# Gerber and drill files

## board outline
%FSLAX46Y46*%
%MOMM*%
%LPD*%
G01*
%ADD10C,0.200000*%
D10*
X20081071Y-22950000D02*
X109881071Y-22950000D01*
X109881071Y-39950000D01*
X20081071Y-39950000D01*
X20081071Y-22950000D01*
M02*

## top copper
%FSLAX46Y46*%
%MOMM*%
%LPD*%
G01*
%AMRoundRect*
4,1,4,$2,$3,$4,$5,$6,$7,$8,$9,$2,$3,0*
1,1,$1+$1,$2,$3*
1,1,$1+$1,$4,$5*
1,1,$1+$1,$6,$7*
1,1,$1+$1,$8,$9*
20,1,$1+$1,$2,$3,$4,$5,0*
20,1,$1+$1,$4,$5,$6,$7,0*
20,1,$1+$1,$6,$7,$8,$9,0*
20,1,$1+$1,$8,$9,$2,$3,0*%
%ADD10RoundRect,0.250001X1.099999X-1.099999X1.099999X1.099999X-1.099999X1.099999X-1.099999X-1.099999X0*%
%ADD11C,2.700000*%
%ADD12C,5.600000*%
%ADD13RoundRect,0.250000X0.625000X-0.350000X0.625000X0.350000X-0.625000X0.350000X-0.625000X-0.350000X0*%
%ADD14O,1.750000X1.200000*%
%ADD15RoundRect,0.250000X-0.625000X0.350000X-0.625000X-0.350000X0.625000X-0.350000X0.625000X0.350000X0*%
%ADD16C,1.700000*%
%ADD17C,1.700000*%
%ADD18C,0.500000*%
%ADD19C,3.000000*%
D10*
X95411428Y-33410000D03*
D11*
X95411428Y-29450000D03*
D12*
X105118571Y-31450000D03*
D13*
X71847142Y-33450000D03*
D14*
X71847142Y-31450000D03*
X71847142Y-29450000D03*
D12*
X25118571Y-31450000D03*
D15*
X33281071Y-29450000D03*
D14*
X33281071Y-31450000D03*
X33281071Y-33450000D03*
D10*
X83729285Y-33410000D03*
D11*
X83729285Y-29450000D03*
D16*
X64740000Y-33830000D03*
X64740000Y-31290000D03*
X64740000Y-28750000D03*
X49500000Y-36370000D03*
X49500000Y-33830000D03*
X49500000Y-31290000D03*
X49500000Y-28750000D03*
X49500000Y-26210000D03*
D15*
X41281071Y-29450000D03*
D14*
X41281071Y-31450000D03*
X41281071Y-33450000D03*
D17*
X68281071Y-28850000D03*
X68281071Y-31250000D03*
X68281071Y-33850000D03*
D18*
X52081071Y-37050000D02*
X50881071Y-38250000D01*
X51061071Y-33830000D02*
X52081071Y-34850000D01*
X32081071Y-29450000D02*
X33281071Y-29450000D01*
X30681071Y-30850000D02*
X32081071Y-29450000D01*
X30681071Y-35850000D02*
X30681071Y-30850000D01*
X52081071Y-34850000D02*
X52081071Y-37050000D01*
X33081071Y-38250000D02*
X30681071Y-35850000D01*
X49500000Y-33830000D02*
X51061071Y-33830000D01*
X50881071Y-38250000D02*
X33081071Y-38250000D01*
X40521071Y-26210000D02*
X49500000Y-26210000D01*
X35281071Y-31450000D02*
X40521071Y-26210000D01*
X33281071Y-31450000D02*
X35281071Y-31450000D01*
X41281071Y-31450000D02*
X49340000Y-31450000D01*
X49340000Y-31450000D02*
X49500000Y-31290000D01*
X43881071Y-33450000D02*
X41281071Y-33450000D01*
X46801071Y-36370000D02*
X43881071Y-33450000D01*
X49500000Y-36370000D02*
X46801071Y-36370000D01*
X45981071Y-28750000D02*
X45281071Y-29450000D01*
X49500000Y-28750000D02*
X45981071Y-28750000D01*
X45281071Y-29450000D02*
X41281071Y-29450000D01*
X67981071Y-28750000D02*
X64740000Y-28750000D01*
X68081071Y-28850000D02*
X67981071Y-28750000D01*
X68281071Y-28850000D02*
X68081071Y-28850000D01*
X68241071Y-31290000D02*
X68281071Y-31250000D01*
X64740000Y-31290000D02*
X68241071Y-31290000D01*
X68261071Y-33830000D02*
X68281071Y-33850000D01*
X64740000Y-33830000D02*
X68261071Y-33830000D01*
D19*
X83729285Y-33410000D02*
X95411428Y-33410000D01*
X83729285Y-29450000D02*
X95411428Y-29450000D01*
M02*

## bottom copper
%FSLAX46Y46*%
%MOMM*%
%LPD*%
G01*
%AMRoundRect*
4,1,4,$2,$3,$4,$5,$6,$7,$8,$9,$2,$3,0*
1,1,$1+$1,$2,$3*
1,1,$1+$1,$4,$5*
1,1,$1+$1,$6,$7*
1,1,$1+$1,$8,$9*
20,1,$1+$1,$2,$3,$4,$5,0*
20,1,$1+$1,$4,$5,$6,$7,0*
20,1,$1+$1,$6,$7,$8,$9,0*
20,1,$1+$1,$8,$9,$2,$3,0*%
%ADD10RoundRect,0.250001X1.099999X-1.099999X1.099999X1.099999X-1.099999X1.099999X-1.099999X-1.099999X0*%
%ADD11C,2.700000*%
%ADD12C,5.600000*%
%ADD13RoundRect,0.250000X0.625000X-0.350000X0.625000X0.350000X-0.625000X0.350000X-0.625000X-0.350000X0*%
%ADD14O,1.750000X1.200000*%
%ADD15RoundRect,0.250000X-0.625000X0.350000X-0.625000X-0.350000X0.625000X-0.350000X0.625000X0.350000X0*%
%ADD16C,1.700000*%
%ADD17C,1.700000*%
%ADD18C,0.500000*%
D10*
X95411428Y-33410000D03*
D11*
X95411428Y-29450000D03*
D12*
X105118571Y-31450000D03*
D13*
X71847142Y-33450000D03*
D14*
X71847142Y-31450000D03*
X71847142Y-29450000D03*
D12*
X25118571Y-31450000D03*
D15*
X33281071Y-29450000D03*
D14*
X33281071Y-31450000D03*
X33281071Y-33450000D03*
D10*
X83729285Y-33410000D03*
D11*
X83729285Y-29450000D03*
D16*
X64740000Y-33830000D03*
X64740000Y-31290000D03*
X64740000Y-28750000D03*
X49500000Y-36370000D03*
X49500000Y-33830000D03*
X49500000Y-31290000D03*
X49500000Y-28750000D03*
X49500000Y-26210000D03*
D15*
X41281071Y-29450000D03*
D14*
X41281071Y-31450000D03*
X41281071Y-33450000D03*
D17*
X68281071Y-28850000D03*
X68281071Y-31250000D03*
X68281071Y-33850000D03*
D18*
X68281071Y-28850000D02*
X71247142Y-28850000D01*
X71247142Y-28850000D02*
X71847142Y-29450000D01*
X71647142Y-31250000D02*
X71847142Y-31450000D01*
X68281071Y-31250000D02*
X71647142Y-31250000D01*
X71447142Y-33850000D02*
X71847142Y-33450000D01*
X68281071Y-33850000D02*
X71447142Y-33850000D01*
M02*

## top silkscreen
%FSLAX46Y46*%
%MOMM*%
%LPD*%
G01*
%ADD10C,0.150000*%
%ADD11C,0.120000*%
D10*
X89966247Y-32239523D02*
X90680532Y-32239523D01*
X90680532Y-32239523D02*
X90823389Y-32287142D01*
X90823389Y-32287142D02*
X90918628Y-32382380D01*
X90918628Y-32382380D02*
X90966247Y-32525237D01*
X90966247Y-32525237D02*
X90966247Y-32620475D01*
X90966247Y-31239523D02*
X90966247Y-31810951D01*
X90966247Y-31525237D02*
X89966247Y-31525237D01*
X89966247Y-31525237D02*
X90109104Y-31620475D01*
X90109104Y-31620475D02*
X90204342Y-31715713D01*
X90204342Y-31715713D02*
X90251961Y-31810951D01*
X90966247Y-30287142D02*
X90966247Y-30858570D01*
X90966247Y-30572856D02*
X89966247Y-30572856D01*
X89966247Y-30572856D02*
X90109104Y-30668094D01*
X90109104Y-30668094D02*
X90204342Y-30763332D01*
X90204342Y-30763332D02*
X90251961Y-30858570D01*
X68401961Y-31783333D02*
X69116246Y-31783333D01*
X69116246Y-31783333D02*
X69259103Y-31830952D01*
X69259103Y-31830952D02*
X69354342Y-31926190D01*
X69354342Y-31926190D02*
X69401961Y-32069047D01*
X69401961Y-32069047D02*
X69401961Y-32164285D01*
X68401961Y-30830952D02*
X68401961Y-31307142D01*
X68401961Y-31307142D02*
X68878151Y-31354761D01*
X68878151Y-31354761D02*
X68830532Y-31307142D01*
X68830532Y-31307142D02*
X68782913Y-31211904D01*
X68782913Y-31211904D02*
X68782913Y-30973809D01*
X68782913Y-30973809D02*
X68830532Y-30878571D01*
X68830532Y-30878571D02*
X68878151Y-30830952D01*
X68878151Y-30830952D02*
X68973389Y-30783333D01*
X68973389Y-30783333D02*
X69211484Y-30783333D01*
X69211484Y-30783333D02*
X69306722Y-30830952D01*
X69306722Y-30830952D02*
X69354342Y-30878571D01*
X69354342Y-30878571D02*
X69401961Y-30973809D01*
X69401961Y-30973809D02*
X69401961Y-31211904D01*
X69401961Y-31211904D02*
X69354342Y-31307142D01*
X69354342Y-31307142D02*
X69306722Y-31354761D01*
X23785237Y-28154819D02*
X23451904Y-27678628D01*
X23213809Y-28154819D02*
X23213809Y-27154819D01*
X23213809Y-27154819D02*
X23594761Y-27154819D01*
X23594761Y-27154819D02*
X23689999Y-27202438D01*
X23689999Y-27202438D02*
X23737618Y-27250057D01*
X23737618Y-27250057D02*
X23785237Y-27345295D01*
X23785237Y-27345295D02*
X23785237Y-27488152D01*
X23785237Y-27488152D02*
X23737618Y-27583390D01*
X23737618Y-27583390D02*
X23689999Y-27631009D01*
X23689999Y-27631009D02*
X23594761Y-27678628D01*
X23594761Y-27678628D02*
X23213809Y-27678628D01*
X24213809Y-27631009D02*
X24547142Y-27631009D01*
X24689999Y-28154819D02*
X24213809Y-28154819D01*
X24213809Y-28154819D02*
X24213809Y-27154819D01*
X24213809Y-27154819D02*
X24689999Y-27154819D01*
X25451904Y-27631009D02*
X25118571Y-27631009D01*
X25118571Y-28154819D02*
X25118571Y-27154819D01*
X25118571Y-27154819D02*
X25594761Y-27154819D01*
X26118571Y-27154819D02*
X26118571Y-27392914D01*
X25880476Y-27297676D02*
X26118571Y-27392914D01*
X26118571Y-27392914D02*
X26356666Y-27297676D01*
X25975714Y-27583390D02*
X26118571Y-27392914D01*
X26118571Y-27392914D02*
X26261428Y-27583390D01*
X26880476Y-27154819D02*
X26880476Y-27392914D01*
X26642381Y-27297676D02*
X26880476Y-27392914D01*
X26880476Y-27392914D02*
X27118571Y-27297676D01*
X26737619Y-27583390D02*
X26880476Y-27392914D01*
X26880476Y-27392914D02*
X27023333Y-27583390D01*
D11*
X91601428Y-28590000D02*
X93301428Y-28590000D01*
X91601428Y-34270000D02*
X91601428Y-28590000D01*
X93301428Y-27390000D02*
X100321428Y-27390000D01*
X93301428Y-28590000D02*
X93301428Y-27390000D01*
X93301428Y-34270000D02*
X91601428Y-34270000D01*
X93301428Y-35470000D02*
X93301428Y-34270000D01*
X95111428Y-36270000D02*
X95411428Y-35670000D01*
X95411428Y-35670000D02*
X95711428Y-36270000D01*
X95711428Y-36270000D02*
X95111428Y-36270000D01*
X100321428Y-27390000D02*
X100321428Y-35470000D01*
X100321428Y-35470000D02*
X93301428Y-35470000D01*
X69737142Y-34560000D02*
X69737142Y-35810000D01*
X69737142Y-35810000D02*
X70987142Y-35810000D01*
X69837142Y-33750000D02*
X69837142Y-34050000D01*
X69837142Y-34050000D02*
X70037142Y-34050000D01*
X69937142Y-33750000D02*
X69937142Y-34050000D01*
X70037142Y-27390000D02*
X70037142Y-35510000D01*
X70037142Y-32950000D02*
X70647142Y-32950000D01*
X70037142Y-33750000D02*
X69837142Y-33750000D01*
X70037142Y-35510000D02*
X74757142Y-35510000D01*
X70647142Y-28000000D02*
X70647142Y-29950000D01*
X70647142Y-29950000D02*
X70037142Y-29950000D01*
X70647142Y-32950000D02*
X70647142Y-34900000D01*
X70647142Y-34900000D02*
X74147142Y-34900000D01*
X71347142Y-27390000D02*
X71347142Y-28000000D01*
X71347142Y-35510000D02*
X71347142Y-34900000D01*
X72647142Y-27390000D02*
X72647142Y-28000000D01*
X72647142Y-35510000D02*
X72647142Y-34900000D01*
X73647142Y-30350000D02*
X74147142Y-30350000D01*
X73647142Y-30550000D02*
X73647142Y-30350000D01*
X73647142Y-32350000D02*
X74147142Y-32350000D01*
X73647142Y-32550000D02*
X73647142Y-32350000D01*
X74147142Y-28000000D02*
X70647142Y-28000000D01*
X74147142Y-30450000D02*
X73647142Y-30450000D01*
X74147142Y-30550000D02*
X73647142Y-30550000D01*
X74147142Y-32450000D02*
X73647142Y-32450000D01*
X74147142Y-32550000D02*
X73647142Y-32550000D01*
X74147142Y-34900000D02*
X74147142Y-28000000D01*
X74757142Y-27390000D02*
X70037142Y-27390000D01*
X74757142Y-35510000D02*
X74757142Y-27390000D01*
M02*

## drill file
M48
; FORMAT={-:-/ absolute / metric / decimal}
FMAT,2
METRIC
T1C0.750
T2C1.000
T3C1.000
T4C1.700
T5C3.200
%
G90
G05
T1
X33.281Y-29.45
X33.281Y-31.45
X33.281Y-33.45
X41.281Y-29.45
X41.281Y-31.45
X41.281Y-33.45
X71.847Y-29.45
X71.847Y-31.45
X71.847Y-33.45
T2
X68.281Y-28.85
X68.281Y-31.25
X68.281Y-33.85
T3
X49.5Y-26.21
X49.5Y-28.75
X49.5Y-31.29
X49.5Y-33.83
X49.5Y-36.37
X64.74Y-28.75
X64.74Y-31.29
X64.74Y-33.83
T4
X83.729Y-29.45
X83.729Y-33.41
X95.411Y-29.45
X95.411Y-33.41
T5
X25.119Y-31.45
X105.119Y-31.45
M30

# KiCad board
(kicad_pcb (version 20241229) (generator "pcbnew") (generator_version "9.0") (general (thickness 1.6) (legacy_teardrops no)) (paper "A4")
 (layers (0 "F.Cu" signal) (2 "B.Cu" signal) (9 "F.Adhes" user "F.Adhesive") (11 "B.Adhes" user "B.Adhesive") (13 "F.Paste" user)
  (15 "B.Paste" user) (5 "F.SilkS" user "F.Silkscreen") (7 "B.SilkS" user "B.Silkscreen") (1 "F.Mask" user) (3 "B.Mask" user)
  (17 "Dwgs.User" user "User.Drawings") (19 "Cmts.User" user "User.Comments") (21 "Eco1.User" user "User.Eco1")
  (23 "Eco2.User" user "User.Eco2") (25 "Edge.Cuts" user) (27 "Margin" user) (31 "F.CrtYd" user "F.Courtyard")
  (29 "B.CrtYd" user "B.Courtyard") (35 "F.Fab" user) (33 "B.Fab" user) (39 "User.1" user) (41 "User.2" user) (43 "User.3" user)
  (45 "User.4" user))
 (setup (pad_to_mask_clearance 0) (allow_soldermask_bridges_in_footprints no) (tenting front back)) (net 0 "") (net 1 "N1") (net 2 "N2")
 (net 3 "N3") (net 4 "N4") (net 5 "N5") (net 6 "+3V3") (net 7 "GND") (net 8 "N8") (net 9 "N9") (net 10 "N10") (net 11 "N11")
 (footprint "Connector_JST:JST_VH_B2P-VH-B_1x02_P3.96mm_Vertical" (layer "F.Cu") (at 95.411428 33.41 90)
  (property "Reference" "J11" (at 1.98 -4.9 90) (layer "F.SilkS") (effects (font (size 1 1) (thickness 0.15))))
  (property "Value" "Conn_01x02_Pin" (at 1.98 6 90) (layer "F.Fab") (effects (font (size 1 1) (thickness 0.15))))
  (fp_line (start 4.82 -3.81) (end 4.82 -2.11) (stroke (width 0.12) (type solid)) (layer "F.SilkS"))
  (fp_line (start -0.86 -3.81) (end 4.82 -3.81) (stroke (width 0.12) (type solid)) (layer "F.SilkS"))
  (fp_line (start 6.02 -2.11) (end 6.02 4.91) (stroke (width 0.12) (type solid)) (layer "F.SilkS"))
  (fp_line (start 4.82 -2.11) (end 6.02 -2.11) (stroke (width 0.12) (type solid)) (layer "F.SilkS"))
  (fp_line (start -0.86 -2.11) (end -0.86 -3.81) (stroke (width 0.12) (type solid)) (layer "F.SilkS"))
  (fp_line (start -2.06 -2.11) (end -0.86 -2.11) (stroke (width 0.12) (type solid)) (layer "F.SilkS"))
  (fp_line (start -2.86 -0.3) (end -2.26 0) (stroke (width 0.12) (type solid)) (layer "F.SilkS"))
  (fp_line (start -2.26 0) (end -2.86 0.3) (stroke (width 0.12) (type solid)) (layer "F.SilkS"))
  (fp_line (start -2.86 0.3) (end -2.86 -0.3) (stroke (width 0.12) (type solid)) (layer "F.SilkS"))
  (fp_line (start 6.02 4.91) (end -2.06 4.91) (stroke (width 0.12) (type solid)) (layer "F.SilkS"))
  (fp_line (start -2.06 4.91) (end -2.06 -2.11) (stroke (width 0.12) (type solid)) (layer "F.SilkS"))
  (pad "1" thru_hole roundrect (at 0 0 90) (size 2.7 2.7) (drill 1.7) (layers "*.Cu" "*.Mask") (remove_unused_layers no)
   (roundrect_rratio 0.092593) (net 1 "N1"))
  (pad "2" thru_hole circle (at 3.96 0 90) (size 2.7 2.7) (drill 1.7) (layers "*.Cu" "*.Mask") (remove_unused_layers no) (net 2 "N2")))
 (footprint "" (layer "F.Cu") (at 105.118571 31.45)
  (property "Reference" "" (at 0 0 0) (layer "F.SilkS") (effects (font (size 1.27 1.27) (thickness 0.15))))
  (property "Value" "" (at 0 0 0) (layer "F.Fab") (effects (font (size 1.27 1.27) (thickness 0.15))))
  (pad "1" thru_hole circle (at 0 0) (size 5.6 5.6) (drill 3.2) (layers "*.Cu" "*.Mask") (remove_unused_layers no) (zone_connect 2)))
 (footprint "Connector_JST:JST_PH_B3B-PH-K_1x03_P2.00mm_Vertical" (layer "F.Cu") (at 71.847142 33.45 90)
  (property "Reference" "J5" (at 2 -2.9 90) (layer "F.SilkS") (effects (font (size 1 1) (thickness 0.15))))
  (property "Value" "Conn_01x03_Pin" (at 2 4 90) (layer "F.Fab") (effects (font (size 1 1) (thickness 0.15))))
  (fp_line (start -1.11 -2.11) (end -2.36 -2.11) (stroke (width 0.12) (type solid)) (layer "F.SilkS"))
  (fp_line (start -2.36 -2.11) (end -2.36 -0.86) (stroke (width 0.12) (type solid)) (layer "F.SilkS"))
  (fp_line (start -0.3 -2.01) (end -0.6 -2.01) (stroke (width 0.12) (type solid)) (layer "F.SilkS"))
  (fp_line (start -0.6 -2.01) (end -0.6 -1.81) (stroke (width 0.12) (type solid)) (layer "F.SilkS"))
  (fp_line (start -0.3 -1.91) (end -0.6 -1.91) (stroke (width 0.12) (type solid)) (layer "F.SilkS"))
  (fp_line (start 6.06 -1.81) (end -2.06 -1.81) (stroke (width 0.12) (type solid)) (layer "F.SilkS"))
  (fp_line (start 0.5 -1.81) (end 0.5 -1.2) (stroke (width 0.12) (type solid)) (layer "F.SilkS"))
  (fp_line (start -0.3 -1.81) (end -0.3 -2.01) (stroke (width 0.12) (type solid)) (layer "F.SilkS"))
  (fp_line (start -2.06 -1.81) (end -2.06 2.91) (stroke (width 0.12) (type solid)) (layer "F.SilkS"))
  (fp_line (start 5.45 -1.2) (end 3.5 -1.2) (stroke (width 0.12) (type solid)) (layer "F.SilkS"))
  (fp_line (start 3.5 -1.2) (end 3.5 -1.81) (stroke (width 0.12) (type solid)) (layer "F.SilkS"))
  (fp_line (start 0.5 -1.2) (end -1.45 -1.2) (stroke (width 0.12) (type solid)) (layer "F.SilkS"))
  (fp_line (start -1.45 -1.2) (end -1.45 2.3) (stroke (width 0.12) (type solid)) (layer "F.SilkS"))
  (fp_line (start 6.06 -0.5) (end 5.45 -0.5) (stroke (width 0.12) (type solid)) (layer "F.SilkS"))
  (fp_line (start -2.06 -0.5) (end -1.45 -0.5) (stroke (width 0.12) (type solid)) (layer "F.SilkS"))
  (fp_line (start 6.06 0.8) (end 5.45 0.8) (stroke (width 0.12) (type solid)) (layer "F.SilkS"))
  (fp_line (start -2.06 0.8) (end -1.45 0.8) (stroke (width 0.12) (type solid)) (layer "F.SilkS"))
  (fp_line (start 3.1 1.8) (end 3.1 2.3) (stroke (width 0.12) (type solid)) (layer "F.SilkS"))
  (fp_line (start 2.9 1.8) (end 3.1 1.8) (stroke (width 0.12) (type solid)) (layer "F.SilkS"))
  (fp_line (start 1.1 1.8) (end 1.1 2.3) (stroke (width 0.12) (type solid)) (layer "F.SilkS"))
  (fp_line (start 0.9 1.8) (end 1.1 1.8) (stroke (width 0.12) (type solid)) (layer "F.SilkS"))
  (fp_line (start 5.45 2.3) (end 5.45 -1.2) (stroke (width 0.12) (type solid)) (layer "F.SilkS"))
  (fp_line (start 3 2.3) (end 3 1.8) (stroke (width 0.12) (type solid)) (layer "F.SilkS"))
  (fp_line (start 2.9 2.3) (end 2.9 1.8) (stroke (width 0.12) (type solid)) (layer "F.SilkS"))
  (fp_line (start 1 2.3) (end 1 1.8) (stroke (width 0.12) (type solid)) (layer "F.SilkS"))
  (fp_line (start 0.9 2.3) (end 0.9 1.8) (stroke (width 0.12) (type solid)) (layer "F.SilkS"))
  (fp_line (start -1.45 2.3) (end 5.45 2.3) (stroke (width 0.12) (type solid)) (layer "F.SilkS"))
  (fp_line (start 6.06 2.91) (end 6.06 -1.81) (stroke (width 0.12) (type solid)) (layer "F.SilkS"))
  (fp_line (start -2.06 2.91) (end 6.06 2.91) (stroke (width 0.12) (type solid)) (layer "F.SilkS"))
  (pad "1" thru_hole roundrect (at 0 0 90) (size 1.2 1.75) (drill 0.75) (layers "*.Cu" "*.Mask") (remove_unused_layers no)
   (roundrect_rratio 0.208333) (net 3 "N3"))
  (pad "2" thru_hole oval (at 2 0 90) (size 1.2 1.75) (drill 0.75) (layers "*.Cu" "*.Mask") (remove_unused_layers no) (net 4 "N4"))
  (pad "3" thru_hole oval (at 4 0 90) (size 1.2 1.75) (drill 0.75) (layers "*.Cu" "*.Mask") (remove_unused_layers no) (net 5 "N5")))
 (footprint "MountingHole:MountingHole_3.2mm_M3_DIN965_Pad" (layer "F.Cu") (at 25.118571 31.45)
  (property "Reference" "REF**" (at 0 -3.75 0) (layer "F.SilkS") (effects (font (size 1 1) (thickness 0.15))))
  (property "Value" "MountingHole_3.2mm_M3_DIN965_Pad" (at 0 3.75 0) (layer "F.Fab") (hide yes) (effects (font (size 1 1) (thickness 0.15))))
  (pad "1" thru_hole circle (at 0 0) (size 5.6 5.6) (drill 3.2) (layers "*.Cu" "*.Mask") (remove_unused_layers no) (zone_connect 2)))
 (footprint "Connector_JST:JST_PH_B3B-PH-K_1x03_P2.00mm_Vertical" (layer "B.Cu") (at 33.281071 29.45 -90)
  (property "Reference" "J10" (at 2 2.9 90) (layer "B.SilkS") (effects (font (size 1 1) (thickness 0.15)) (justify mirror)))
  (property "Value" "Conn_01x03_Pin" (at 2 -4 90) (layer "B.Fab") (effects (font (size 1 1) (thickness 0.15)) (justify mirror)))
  (pad "1" thru_hole roundrect (at 0 0 270) (size 1.2 1.75) (drill 0.75) (layers "*.Cu" "*.Mask") (remove_unused_layers no)
   (roundrect_rratio 0.208333) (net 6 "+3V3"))
  (pad "2" thru_hole oval (at 2 0 270) (size 1.2 1.75) (drill 0.75) (layers "*.Cu" "*.Mask") (remove_unused_layers no) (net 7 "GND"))
  (pad "3" thru_hole oval (at 4 0 270) (size 1.2 1.75) (drill 0.75) (layers "*.Cu" "*.Mask") (remove_unused_layers no) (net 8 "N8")))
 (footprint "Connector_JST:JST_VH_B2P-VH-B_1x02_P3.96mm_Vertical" (layer "B.Cu") (at 83.729285 33.41 90)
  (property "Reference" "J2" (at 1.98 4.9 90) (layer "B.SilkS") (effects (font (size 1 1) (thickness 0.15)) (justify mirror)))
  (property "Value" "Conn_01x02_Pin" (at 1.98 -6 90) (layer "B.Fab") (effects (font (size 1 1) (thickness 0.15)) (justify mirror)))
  (pad "1" thru_hole roundrect (at 0 0 90) (size 2.7 2.7) (drill 1.7) (layers "*.Cu" "*.Mask") (remove_unused_layers no)
   (roundrect_rratio 0.092593) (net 1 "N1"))
  (pad "2" thru_hole circle (at 3.96 0 90) (size 2.7 2.7) (drill 1.7) (layers "*.Cu" "*.Mask") (remove_unused_layers no) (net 2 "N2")))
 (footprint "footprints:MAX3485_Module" (layer "B.Cu") (at 60.74 26.79 90)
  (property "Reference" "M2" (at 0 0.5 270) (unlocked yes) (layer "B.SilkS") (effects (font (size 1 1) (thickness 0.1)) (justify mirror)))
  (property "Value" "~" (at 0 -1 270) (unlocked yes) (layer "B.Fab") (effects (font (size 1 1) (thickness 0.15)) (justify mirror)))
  (pad "1" thru_hole circle (at -7.04 4 90) (size 1.7 1.7) (drill 1) (layers "*.Cu" "*.Mask") (remove_unused_layers no) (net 3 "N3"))
  (pad "2" thru_hole circle (at -4.5 4 90) (size 1.7 1.7) (drill 1) (layers "*.Cu" "*.Mask") (remove_unused_layers no) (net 4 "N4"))
  (pad "3" thru_hole circle (at -1.96 4 90) (size 1.7 1.7) (drill 1) (layers "*.Cu" "*.Mask") (remove_unused_layers no) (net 5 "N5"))
  (pad "4" thru_hole circle (at -9.58 -11.24 90) (size 1.7 1.7) (drill 1) (layers "*.Cu" "*.Mask") (remove_unused_layers no) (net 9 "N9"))
  (pad "5" thru_hole circle (at -7.04 -11.24 90) (size 1.7 1.7) (drill 1) (layers "*.Cu" "*.Mask") (remove_unused_layers no) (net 6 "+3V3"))
  (pad "6" thru_hole circle (at -4.5 -11.24 90) (size 1.7 1.7) (drill 1) (layers "*.Cu" "*.Mask") (remove_unused_layers no) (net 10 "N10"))
  (pad "7" thru_hole circle (at -1.96 -11.24 90) (size 1.7 1.7) (drill 1) (layers "*.Cu" "*.Mask") (remove_unused_layers no) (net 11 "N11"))
  (pad "8" thru_hole circle (at 0.58 -11.24 90) (size 1.7 1.7) (drill 1) (layers "*.Cu" "*.Mask") (remove_unused_layers no) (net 7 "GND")))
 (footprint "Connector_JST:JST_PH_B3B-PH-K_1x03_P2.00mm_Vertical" (layer "B.Cu") (at 41.281071 29.45 -90)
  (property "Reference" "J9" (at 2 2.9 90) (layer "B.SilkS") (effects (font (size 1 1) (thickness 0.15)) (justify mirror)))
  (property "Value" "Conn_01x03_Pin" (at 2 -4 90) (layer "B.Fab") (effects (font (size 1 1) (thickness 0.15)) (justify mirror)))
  (pad "1" thru_hole roundrect (at 0 0 270) (size 1.2 1.75) (drill 0.75) (layers "*.Cu" "*.Mask") (remove_unused_layers no)
   (roundrect_rratio 0.208333) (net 11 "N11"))
  (pad "2" thru_hole oval (at 2 0 270) (size 1.2 1.75) (drill 0.75) (layers "*.Cu" "*.Mask") (remove_unused_layers no) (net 10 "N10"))
  (pad "3" thru_hole oval (at 4 0 270) (size 1.2 1.75) (drill 0.75) (layers "*.Cu" "*.Mask") (remove_unused_layers no) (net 9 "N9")))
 (gr_rect (start 20.081071 22.95) (end 109.881071 39.95) (stroke (width 0.2) (type solid)) (fill no) (layer "Edge.Cuts"))
 (segment (start 52.081071 37.05) (end 50.881071 38.25) (width 0.5) (layer "F.Cu") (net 6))
 (segment (start 51.061071 33.83) (end 52.081071 34.85) (width 0.5) (layer "F.Cu") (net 6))
 (segment (start 32.081071 29.45) (end 33.281071 29.45) (width 0.5) (layer "F.Cu") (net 6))
 (segment (start 30.681071 30.85) (end 32.081071 29.45) (width 0.5) (layer "F.Cu") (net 6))
 (segment (start 30.681071 35.85) (end 30.681071 30.85) (width 0.5) (layer "F.Cu") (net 6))
 (segment (start 52.081071 34.85) (end 52.081071 37.05) (width 0.5) (layer "F.Cu") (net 6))
 (segment (start 33.081071 38.25) (end 30.681071 35.85) (width 0.5) (layer "F.Cu") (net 6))
 (segment (start 49.5 33.83) (end 51.061071 33.83) (width 0.5) (layer "F.Cu") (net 6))
 (segment (start 50.881071 38.25) (end 33.081071 38.25) (width 0.5) (layer "F.Cu") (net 6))
 (segment (start 40.521071 26.21) (end 49.5 26.21) (width 0.5) (layer "F.Cu") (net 7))
 (segment (start 35.281071 31.45) (end 40.521071 26.21) (width 0.5) (layer "F.Cu") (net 7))
 (segment (start 33.281071 31.45) (end 35.281071 31.45) (width 0.5) (layer "F.Cu") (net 7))
 (segment (start 41.281071 31.45) (end 49.34 31.45) (width 0.5) (layer "F.Cu") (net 10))
 (segment (start 49.34 31.45) (end 49.5 31.29) (width 0.5) (layer "F.Cu") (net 10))
 (segment (start 43.881071 33.45) (end 41.281071 33.45) (width 0.5) (layer "F.Cu") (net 9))
 (segment (start 46.801071 36.37) (end 43.881071 33.45) (width 0.5) (layer "F.Cu") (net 9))
 (segment (start 49.5 36.37) (end 46.801071 36.37) (width 0.5) (layer "F.Cu") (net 9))
 (segment (start 45.981071 28.75) (end 45.281071 29.45) (width 0.5) (layer "F.Cu") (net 11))
 (segment (start 49.5 28.75) (end 45.981071 28.75) (width 0.5) (layer "F.Cu") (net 11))
 (segment (start 45.281071 29.45) (end 41.281071 29.45) (width 0.5) (layer "F.Cu") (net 11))
 (segment (start 67.981071 28.75) (end 64.74 28.75) (width 0.5) (layer "F.Cu") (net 5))
 (segment (start 68.081071 28.85) (end 67.981071 28.75) (width 0.5) (layer "F.Cu") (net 5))
 (segment (start 68.281071 28.85) (end 68.081071 28.85) (width 0.5) (layer "F.Cu") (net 5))
 (via (at 68.281071 28.85) (size 1.7) (drill 1) (layers "F.Cu" "B.Cu") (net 5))
 (segment (start 68.281071 28.85) (end 71.247142 28.85) (width 0.5) (layer "B.Cu") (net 5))
 (segment (start 71.247142 28.85) (end 71.847142 29.45) (width 0.5) (layer "B.Cu") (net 5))
 (segment (start 68.241071 31.29) (end 68.281071 31.25) (width 0.5) (layer "F.Cu") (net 4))
 (segment (start 64.74 31.29) (end 68.241071 31.29) (width 0.5) (layer "F.Cu") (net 4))
 (via (at 68.281071 31.25) (size 1.7) (drill 1) (layers "F.Cu" "B.Cu") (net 4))
 (segment (start 71.647142 31.25) (end 71.847142 31.45) (width 0.5) (layer "B.Cu") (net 4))
 (segment (start 68.281071 31.25) (end 71.647142 31.25) (width 0.5) (layer "B.Cu") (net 4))
 (segment (start 68.261071 33.83) (end 68.281071 33.85) (width 0.5) (layer "F.Cu") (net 3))
 (segment (start 64.74 33.83) (end 68.261071 33.83) (width 0.5) (layer "F.Cu") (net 3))
 (via (at 68.281071 33.85) (size 1.7) (drill 1) (layers "F.Cu" "B.Cu") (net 3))
 (segment (start 71.447142 33.85) (end 71.847142 33.45) (width 0.5) (layer "B.Cu") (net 3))
 (segment (start 68.281071 33.85) (end 71.447142 33.85) (width 0.5) (layer "B.Cu") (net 3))
 (segment (start 83.729285 33.41) (end 95.411428 33.41) (width 3) (layer "F.Cu") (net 1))
 (segment (start 83.729285 29.45) (end 95.411428 29.45) (width 3) (layer "F.Cu") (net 2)))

